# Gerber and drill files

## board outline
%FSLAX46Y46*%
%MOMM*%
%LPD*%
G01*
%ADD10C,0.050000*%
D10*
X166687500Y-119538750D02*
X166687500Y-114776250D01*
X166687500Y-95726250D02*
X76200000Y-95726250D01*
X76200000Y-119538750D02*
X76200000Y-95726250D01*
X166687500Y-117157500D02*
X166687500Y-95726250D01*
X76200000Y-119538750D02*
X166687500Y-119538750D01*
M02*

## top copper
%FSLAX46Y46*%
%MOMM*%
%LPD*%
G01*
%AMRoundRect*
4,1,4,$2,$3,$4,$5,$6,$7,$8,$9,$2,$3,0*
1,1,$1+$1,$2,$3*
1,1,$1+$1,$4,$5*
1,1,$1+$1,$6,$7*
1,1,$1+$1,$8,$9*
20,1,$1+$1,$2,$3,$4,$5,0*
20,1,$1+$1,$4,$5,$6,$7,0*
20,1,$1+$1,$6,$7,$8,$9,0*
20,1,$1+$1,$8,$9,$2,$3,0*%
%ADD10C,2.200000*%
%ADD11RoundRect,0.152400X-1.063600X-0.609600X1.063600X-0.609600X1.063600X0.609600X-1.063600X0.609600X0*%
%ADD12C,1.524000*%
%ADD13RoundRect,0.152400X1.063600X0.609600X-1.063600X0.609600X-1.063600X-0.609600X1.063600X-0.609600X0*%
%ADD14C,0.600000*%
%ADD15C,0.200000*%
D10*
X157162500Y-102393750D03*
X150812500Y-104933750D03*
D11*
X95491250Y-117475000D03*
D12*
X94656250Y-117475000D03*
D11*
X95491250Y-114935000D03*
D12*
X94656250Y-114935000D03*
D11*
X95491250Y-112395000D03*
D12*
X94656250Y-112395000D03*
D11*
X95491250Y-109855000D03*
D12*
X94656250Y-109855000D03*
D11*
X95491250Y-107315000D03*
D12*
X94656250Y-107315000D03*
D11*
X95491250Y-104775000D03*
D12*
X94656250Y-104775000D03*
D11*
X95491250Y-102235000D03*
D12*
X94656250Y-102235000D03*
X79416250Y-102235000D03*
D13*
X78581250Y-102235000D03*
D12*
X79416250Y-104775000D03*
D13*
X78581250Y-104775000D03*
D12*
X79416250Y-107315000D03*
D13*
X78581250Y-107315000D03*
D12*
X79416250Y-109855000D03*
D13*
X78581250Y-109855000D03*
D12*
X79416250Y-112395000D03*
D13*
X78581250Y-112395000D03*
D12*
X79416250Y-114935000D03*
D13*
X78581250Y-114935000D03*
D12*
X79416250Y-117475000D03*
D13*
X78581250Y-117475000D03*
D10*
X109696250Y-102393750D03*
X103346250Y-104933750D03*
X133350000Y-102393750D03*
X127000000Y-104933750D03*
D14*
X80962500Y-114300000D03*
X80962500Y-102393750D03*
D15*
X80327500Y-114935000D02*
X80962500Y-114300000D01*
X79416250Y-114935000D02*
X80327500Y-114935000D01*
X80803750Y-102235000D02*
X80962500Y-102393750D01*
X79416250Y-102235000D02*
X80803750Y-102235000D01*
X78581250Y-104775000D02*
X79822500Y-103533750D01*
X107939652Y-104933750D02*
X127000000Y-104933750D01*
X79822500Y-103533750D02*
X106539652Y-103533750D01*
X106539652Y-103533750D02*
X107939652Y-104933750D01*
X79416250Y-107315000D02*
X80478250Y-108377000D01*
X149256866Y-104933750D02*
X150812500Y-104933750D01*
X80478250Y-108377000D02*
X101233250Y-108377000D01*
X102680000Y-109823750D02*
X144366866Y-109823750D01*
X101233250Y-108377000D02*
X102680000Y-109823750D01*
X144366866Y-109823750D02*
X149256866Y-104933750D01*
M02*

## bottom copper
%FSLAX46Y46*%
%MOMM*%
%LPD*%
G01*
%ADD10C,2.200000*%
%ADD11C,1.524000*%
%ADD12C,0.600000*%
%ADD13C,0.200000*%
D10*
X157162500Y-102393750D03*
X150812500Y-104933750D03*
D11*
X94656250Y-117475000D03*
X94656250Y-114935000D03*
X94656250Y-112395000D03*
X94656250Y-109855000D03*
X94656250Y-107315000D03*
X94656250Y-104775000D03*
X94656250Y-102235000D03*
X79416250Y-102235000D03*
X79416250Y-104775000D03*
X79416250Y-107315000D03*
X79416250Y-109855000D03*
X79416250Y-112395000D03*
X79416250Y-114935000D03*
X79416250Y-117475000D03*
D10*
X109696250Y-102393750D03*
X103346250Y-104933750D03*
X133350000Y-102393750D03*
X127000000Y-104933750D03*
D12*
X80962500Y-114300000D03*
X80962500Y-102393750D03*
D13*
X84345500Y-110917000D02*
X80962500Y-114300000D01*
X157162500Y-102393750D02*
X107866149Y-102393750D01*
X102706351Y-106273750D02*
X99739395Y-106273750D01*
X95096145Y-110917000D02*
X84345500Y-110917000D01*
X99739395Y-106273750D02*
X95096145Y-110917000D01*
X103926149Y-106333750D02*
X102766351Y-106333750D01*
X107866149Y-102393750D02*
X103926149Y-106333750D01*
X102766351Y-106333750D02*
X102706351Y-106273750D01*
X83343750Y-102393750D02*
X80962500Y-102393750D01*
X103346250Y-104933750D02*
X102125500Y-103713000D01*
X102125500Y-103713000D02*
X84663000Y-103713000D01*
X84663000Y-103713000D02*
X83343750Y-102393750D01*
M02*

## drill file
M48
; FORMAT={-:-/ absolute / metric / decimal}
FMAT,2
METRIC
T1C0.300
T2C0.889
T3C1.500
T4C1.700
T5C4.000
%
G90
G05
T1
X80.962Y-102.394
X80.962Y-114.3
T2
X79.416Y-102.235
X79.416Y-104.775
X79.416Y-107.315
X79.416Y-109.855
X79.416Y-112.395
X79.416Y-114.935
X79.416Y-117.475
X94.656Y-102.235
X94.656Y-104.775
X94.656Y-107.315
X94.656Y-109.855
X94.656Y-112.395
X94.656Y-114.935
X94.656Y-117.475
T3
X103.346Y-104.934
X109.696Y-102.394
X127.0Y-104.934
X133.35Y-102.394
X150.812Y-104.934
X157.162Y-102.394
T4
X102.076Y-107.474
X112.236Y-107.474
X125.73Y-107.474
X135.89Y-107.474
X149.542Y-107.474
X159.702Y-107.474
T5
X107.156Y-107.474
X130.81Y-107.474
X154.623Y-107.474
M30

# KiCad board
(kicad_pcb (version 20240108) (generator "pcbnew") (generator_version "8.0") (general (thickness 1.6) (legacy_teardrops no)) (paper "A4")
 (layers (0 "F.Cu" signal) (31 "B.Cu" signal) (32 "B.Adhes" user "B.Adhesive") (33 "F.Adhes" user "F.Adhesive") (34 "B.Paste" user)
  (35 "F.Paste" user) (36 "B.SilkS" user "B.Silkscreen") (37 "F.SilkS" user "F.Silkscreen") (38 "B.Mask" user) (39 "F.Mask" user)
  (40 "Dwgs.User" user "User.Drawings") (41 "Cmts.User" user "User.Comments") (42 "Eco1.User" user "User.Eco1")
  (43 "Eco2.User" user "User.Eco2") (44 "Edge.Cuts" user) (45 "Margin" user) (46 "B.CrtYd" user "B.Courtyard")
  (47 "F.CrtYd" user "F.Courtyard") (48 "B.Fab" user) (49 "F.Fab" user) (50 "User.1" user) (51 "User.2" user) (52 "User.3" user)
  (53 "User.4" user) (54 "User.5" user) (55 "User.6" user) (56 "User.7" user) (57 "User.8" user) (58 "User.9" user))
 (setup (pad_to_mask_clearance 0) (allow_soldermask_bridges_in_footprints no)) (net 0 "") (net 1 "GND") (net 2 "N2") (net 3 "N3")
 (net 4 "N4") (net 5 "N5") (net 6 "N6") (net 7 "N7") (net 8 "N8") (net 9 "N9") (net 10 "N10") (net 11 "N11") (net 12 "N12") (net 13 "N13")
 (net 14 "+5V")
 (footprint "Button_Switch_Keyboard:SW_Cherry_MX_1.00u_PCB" (layer "F.Cu") (at 157.1625 102.39375)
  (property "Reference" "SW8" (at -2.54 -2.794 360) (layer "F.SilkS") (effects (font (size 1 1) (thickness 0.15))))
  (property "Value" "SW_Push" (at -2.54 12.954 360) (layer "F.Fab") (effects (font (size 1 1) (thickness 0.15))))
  (pad "" np_thru_hole circle (at -7.62 5.08) (size 1.7 1.7) (drill 1.7) (layers "*.Cu" "*.Mask"))
  (pad "" np_thru_hole circle (at -2.54 5.08) (size 4 4) (drill 4) (layers "*.Cu" "*.Mask"))
  (pad "" np_thru_hole circle (at 2.54 5.08) (size 1.7 1.7) (drill 1.7) (layers "*.Cu" "*.Mask"))
  (pad "1" thru_hole circle (at 0 0) (size 2.2 2.2) (drill 1.5) (layers "*.Cu" "*.Mask") (remove_unused_layers no) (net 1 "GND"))
  (pad "2" thru_hole circle (at -6.35 2.54) (size 2.2 2.2) (drill 1.5) (layers "*.Cu" "*.Mask") (remove_unused_layers no) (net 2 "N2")))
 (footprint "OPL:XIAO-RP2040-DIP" (layer "F.Cu") (at 87.03625 109.855 180)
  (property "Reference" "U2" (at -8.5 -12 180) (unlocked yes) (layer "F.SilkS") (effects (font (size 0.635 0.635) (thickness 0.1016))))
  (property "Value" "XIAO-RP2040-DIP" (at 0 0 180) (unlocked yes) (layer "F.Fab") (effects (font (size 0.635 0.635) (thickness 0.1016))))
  (pad "1" smd roundrect (at -8.455 -7.62) (size 2.432 1.524) (layers "F.Cu" "F.Mask") (roundrect_rratio 0.1) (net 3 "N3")
   (thermal_bridge_angle 45))
  (pad "1" thru_hole circle (at -7.62 -7.62) (size 1.524 1.524) (drill 0.889) (layers "*.Cu" "*.Mask") (remove_unused_layers no)
   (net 3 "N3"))
  (pad "2" smd roundrect (at -8.455 -5.08) (size 2.432 1.524) (layers "F.Cu" "F.Mask") (roundrect_rratio 0.1) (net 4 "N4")
   (thermal_bridge_angle 45))
  (pad "2" thru_hole circle (at -7.62 -5.08) (size 1.524 1.524) (drill 0.889) (layers "*.Cu" "*.Mask") (remove_unused_layers no)
   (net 4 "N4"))
  (pad "3" smd roundrect (at -8.455 -2.54) (size 2.432 1.524) (layers "F.Cu" "F.Mask") (roundrect_rratio 0.1) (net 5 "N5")
   (thermal_bridge_angle 45))
  (pad "3" thru_hole circle (at -7.62 -2.54) (size 1.524 1.524) (drill 0.889) (layers "*.Cu" "*.Mask") (remove_unused_layers no)
   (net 5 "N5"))
  (pad "4" smd roundrect (at -8.455 0) (size 2.432 1.524) (layers "F.Cu" "F.Mask") (roundrect_rratio 0.1) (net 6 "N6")
   (thermal_bridge_angle 45))
  (pad "4" thru_hole circle (at -7.62 0) (size 1.524 1.524) (drill 0.889) (layers "*.Cu" "*.Mask") (remove_unused_layers no) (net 6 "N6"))
  (pad "5" smd roundrect (at -8.455 2.54) (size 2.432 1.524) (layers "F.Cu" "F.Mask") (roundrect_rratio 0.1) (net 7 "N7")
   (thermal_bridge_angle 45))
  (pad "5" thru_hole circle (at -7.62 2.54) (size 1.524 1.524) (drill 0.889) (layers "*.Cu" "*.Mask") (remove_unused_layers no) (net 7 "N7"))
  (pad "6" smd roundrect (at -8.455 5.08) (size 2.432 1.524) (layers "F.Cu" "F.Mask") (roundrect_rratio 0.1) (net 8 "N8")
   (thermal_bridge_angle 45))
  (pad "6" thru_hole circle (at -7.62 5.08) (size 1.524 1.524) (drill 0.889) (layers "*.Cu" "*.Mask") (remove_unused_layers no) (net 8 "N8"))
  (pad "7" smd roundrect (at -8.455 7.62) (size 2.432 1.524) (layers "F.Cu" "F.Mask") (roundrect_rratio 0.1) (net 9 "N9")
   (thermal_bridge_angle 45))
  (pad "7" thru_hole circle (at -7.62 7.62) (size 1.524 1.524) (drill 0.889) (layers "*.Cu" "*.Mask") (remove_unused_layers no) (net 9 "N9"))
  (pad "8" thru_hole circle (at 7.62 7.62 180) (size 1.524 1.524) (drill 0.889) (layers "*.Cu" "*.Mask") (remove_unused_layers no)
   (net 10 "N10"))
  (pad "8" smd roundrect (at 8.455 7.62 180) (size 2.432 1.524) (layers "F.Cu" "F.Mask") (roundrect_rratio 0.1) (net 10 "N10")
   (thermal_bridge_angle 45))
  (pad "9" thru_hole circle (at 7.62 5.08 180) (size 1.524 1.524) (drill 0.889) (layers "*.Cu" "*.Mask") (remove_unused_layers no)
   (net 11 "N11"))
  (pad "9" smd roundrect (at 8.455 5.08 180) (size 2.432 1.524) (layers "F.Cu" "F.Mask") (roundrect_rratio 0.1) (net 11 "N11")
   (thermal_bridge_angle 45))
  (pad "10" thru_hole circle (at 7.62 2.54 180) (size 1.524 1.524) (drill 0.889) (layers "*.Cu" "*.Mask") (remove_unused_layers no)
   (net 2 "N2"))
  (pad "10" smd roundrect (at 8.455 2.54 180) (size 2.432 1.524) (layers "F.Cu" "F.Mask") (roundrect_rratio 0.1) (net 2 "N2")
   (thermal_bridge_angle 45))
  (pad "11" thru_hole circle (at 7.62 0 180) (size 1.524 1.524) (drill 0.889) (layers "*.Cu" "*.Mask") (remove_unused_layers no)
   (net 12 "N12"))
  (pad "11" smd roundrect (at 8.455 0 180) (size 2.432 1.524) (layers "F.Cu" "F.Mask") (roundrect_rratio 0.1) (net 12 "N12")
   (thermal_bridge_angle 45))
  (pad "12" thru_hole circle (at 7.62 -2.54 180) (size 1.524 1.524) (drill 0.889) (layers "*.Cu" "*.Mask") (remove_unused_layers no)
   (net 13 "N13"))
  (pad "12" smd roundrect (at 8.455 -2.54 180) (size 2.432 1.524) (layers "F.Cu" "F.Mask") (roundrect_rratio 0.1) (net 13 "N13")
   (thermal_bridge_angle 45))
  (pad "13" thru_hole circle (at 7.62 -5.08 180) (size 1.524 1.524) (drill 0.889) (layers "*.Cu" "*.Mask") (remove_unused_layers no)
   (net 1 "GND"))
  (pad "13" smd roundrect (at 8.455 -5.08 180) (size 2.432 1.524) (layers "F.Cu" "F.Mask") (roundrect_rratio 0.1) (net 1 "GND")
   (thermal_bridge_angle 45))
  (pad "14" thru_hole circle (at 7.62 -7.62 180) (size 1.524 1.524) (drill 0.889) (layers "*.Cu" "*.Mask") (remove_unused_layers no)
   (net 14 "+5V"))
  (pad "14" smd roundrect (at 8.455 -7.62 180) (size 2.432 1.524) (layers "F.Cu" "F.Mask") (roundrect_rratio 0.1) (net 14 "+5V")
   (thermal_bridge_angle 45)))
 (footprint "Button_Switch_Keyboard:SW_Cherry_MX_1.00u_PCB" (layer "F.Cu") (at 109.69625 102.39375)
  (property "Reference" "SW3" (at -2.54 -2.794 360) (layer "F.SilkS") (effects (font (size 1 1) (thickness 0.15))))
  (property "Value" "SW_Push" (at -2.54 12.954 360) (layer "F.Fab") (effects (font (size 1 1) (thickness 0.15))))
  (pad "" np_thru_hole circle (at -7.62 5.08) (size 1.7 1.7) (drill 1.7) (layers "*.Cu" "*.Mask"))
  (pad "" np_thru_hole circle (at -2.54 5.08) (size 4 4) (drill 4) (layers "*.Cu" "*.Mask"))
  (pad "" np_thru_hole circle (at 2.54 5.08) (size 1.7 1.7) (drill 1.7) (layers "*.Cu" "*.Mask"))
  (pad "1" thru_hole circle (at 0 0) (size 2.2 2.2) (drill 1.5) (layers "*.Cu" "*.Mask") (remove_unused_layers no) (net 1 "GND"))
  (pad "2" thru_hole circle (at -6.35 2.54) (size 2.2 2.2) (drill 1.5) (layers "*.Cu" "*.Mask") (remove_unused_layers no) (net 10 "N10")))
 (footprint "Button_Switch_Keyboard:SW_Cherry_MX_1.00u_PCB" (layer "F.Cu") (at 133.35 102.39375)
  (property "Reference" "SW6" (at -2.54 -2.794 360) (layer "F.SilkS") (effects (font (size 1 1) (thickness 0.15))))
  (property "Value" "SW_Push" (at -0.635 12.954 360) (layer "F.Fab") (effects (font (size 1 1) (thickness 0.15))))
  (pad "" np_thru_hole circle (at -7.62 5.08) (size 1.7 1.7) (drill 1.7) (layers "*.Cu" "*.Mask"))
  (pad "" np_thru_hole circle (at -2.54 5.08) (size 4 4) (drill 4) (layers "*.Cu" "*.Mask"))
  (pad "" np_thru_hole circle (at 2.54 5.08) (size 1.7 1.7) (drill 1.7) (layers "*.Cu" "*.Mask"))
  (pad "1" thru_hole circle (at 0 0) (size 2.2 2.2) (drill 1.5) (layers "*.Cu" "*.Mask") (remove_unused_layers no) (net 1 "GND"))
  (pad "2" thru_hole circle (at -6.35 2.54) (size 2.2 2.2) (drill 1.5) (layers "*.Cu" "*.Mask") (remove_unused_layers no) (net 11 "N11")))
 (gr_line (start 166.6875 119.53875) (end 166.6875 114.77625) (stroke (width 0.05) (type default)) (layer "Edge.Cuts"))
 (gr_line (start 166.6875 95.72625) (end 76.2 95.72625) (stroke (width 0.05) (type default)) (layer "Edge.Cuts"))
 (gr_line (start 76.2 119.53875) (end 76.2 95.72625) (stroke (width 0.05) (type default)) (layer "Edge.Cuts"))
 (gr_line (start 166.6875 117.1575) (end 166.6875 95.72625) (stroke (width 0.05) (type default)) (layer "Edge.Cuts"))
 (gr_line (start 76.2 119.53875) (end 166.6875 119.53875) (stroke (width 0.05) (type default)) (layer "Edge.Cuts"))
 (segment (start 80.3275 114.935) (end 80.9625 114.3) (width 0.2) (layer "F.Cu") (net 1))
 (segment (start 79.41625 114.935) (end 80.3275 114.935) (width 0.2) (layer "F.Cu") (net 1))
 (via (at 80.9625 114.3) (size 0.6) (drill 0.3) (layers "F.Cu" "B.Cu") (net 1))
 (segment (start 84.3455 110.917) (end 80.9625 114.3) (width 0.2) (layer "B.Cu") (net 1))
 (segment (start 157.1625 102.39375) (end 107.866149 102.39375) (width 0.2) (layer "B.Cu") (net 1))
 (segment (start 102.706351 106.27375) (end 99.739395 106.27375) (width 0.2) (layer "B.Cu") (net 1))
 (segment (start 95.096145 110.917) (end 84.3455 110.917) (width 0.2) (layer "B.Cu") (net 1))
 (segment (start 99.739395 106.27375) (end 95.096145 110.917) (width 0.2) (layer "B.Cu") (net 1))
 (segment (start 103.926149 106.33375) (end 102.766351 106.33375) (width 0.2) (layer "B.Cu") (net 1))
 (segment (start 107.866149 102.39375) (end 103.926149 106.33375) (width 0.2) (layer "B.Cu") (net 1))
 (segment (start 102.766351 106.33375) (end 102.706351 106.27375) (width 0.2) (layer "B.Cu") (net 1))
 (segment (start 80.80375 102.235) (end 80.9625 102.39375) (width 0.2) (layer "F.Cu") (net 10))
 (segment (start 79.41625 102.235) (end 80.80375 102.235) (width 0.2) (layer "F.Cu") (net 10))
 (via (at 80.9625 102.39375) (size 0.6) (drill 0.3) (layers "F.Cu" "B.Cu") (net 10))
 (segment (start 83.34375 102.39375) (end 80.9625 102.39375) (width 0.2) (layer "B.Cu") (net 10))
 (segment (start 103.34625 104.93375) (end 102.1255 103.713) (width 0.2) (layer "B.Cu") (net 10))
 (segment (start 102.1255 103.713) (end 84.663 103.713) (width 0.2) (layer "B.Cu") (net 10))
 (segment (start 84.663 103.713) (end 83.34375 102.39375) (width 0.2) (layer "B.Cu") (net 10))
 (segment (start 78.58125 104.775) (end 79.8225 103.53375) (width 0.2) (layer "F.Cu") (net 11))
 (segment (start 107.939652 104.93375) (end 127 104.93375) (width 0.2) (layer "F.Cu") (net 11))
 (segment (start 79.8225 103.53375) (end 106.539652 103.53375) (width 0.2) (layer "F.Cu") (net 11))
 (segment (start 106.539652 103.53375) (end 107.939652 104.93375) (width 0.2) (layer "F.Cu") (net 11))
 (segment (start 79.41625 107.315) (end 80.47825 108.377) (width 0.2) (layer "F.Cu") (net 2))
 (segment (start 149.256866 104.93375) (end 150.8125 104.93375) (width 0.2) (layer "F.Cu") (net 2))
 (segment (start 80.47825 108.377) (end 101.23325 108.377) (width 0.2) (layer "F.Cu") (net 2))
 (segment (start 102.68 109.82375) (end 144.366866 109.82375) (width 0.2) (layer "F.Cu") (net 2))
 (segment (start 101.23325 108.377) (end 102.68 109.82375) (width 0.2) (layer "F.Cu") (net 2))
 (segment (start 144.366866 109.82375) (end 149.256866 104.93375) (width 0.2) (layer "F.Cu") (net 2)))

